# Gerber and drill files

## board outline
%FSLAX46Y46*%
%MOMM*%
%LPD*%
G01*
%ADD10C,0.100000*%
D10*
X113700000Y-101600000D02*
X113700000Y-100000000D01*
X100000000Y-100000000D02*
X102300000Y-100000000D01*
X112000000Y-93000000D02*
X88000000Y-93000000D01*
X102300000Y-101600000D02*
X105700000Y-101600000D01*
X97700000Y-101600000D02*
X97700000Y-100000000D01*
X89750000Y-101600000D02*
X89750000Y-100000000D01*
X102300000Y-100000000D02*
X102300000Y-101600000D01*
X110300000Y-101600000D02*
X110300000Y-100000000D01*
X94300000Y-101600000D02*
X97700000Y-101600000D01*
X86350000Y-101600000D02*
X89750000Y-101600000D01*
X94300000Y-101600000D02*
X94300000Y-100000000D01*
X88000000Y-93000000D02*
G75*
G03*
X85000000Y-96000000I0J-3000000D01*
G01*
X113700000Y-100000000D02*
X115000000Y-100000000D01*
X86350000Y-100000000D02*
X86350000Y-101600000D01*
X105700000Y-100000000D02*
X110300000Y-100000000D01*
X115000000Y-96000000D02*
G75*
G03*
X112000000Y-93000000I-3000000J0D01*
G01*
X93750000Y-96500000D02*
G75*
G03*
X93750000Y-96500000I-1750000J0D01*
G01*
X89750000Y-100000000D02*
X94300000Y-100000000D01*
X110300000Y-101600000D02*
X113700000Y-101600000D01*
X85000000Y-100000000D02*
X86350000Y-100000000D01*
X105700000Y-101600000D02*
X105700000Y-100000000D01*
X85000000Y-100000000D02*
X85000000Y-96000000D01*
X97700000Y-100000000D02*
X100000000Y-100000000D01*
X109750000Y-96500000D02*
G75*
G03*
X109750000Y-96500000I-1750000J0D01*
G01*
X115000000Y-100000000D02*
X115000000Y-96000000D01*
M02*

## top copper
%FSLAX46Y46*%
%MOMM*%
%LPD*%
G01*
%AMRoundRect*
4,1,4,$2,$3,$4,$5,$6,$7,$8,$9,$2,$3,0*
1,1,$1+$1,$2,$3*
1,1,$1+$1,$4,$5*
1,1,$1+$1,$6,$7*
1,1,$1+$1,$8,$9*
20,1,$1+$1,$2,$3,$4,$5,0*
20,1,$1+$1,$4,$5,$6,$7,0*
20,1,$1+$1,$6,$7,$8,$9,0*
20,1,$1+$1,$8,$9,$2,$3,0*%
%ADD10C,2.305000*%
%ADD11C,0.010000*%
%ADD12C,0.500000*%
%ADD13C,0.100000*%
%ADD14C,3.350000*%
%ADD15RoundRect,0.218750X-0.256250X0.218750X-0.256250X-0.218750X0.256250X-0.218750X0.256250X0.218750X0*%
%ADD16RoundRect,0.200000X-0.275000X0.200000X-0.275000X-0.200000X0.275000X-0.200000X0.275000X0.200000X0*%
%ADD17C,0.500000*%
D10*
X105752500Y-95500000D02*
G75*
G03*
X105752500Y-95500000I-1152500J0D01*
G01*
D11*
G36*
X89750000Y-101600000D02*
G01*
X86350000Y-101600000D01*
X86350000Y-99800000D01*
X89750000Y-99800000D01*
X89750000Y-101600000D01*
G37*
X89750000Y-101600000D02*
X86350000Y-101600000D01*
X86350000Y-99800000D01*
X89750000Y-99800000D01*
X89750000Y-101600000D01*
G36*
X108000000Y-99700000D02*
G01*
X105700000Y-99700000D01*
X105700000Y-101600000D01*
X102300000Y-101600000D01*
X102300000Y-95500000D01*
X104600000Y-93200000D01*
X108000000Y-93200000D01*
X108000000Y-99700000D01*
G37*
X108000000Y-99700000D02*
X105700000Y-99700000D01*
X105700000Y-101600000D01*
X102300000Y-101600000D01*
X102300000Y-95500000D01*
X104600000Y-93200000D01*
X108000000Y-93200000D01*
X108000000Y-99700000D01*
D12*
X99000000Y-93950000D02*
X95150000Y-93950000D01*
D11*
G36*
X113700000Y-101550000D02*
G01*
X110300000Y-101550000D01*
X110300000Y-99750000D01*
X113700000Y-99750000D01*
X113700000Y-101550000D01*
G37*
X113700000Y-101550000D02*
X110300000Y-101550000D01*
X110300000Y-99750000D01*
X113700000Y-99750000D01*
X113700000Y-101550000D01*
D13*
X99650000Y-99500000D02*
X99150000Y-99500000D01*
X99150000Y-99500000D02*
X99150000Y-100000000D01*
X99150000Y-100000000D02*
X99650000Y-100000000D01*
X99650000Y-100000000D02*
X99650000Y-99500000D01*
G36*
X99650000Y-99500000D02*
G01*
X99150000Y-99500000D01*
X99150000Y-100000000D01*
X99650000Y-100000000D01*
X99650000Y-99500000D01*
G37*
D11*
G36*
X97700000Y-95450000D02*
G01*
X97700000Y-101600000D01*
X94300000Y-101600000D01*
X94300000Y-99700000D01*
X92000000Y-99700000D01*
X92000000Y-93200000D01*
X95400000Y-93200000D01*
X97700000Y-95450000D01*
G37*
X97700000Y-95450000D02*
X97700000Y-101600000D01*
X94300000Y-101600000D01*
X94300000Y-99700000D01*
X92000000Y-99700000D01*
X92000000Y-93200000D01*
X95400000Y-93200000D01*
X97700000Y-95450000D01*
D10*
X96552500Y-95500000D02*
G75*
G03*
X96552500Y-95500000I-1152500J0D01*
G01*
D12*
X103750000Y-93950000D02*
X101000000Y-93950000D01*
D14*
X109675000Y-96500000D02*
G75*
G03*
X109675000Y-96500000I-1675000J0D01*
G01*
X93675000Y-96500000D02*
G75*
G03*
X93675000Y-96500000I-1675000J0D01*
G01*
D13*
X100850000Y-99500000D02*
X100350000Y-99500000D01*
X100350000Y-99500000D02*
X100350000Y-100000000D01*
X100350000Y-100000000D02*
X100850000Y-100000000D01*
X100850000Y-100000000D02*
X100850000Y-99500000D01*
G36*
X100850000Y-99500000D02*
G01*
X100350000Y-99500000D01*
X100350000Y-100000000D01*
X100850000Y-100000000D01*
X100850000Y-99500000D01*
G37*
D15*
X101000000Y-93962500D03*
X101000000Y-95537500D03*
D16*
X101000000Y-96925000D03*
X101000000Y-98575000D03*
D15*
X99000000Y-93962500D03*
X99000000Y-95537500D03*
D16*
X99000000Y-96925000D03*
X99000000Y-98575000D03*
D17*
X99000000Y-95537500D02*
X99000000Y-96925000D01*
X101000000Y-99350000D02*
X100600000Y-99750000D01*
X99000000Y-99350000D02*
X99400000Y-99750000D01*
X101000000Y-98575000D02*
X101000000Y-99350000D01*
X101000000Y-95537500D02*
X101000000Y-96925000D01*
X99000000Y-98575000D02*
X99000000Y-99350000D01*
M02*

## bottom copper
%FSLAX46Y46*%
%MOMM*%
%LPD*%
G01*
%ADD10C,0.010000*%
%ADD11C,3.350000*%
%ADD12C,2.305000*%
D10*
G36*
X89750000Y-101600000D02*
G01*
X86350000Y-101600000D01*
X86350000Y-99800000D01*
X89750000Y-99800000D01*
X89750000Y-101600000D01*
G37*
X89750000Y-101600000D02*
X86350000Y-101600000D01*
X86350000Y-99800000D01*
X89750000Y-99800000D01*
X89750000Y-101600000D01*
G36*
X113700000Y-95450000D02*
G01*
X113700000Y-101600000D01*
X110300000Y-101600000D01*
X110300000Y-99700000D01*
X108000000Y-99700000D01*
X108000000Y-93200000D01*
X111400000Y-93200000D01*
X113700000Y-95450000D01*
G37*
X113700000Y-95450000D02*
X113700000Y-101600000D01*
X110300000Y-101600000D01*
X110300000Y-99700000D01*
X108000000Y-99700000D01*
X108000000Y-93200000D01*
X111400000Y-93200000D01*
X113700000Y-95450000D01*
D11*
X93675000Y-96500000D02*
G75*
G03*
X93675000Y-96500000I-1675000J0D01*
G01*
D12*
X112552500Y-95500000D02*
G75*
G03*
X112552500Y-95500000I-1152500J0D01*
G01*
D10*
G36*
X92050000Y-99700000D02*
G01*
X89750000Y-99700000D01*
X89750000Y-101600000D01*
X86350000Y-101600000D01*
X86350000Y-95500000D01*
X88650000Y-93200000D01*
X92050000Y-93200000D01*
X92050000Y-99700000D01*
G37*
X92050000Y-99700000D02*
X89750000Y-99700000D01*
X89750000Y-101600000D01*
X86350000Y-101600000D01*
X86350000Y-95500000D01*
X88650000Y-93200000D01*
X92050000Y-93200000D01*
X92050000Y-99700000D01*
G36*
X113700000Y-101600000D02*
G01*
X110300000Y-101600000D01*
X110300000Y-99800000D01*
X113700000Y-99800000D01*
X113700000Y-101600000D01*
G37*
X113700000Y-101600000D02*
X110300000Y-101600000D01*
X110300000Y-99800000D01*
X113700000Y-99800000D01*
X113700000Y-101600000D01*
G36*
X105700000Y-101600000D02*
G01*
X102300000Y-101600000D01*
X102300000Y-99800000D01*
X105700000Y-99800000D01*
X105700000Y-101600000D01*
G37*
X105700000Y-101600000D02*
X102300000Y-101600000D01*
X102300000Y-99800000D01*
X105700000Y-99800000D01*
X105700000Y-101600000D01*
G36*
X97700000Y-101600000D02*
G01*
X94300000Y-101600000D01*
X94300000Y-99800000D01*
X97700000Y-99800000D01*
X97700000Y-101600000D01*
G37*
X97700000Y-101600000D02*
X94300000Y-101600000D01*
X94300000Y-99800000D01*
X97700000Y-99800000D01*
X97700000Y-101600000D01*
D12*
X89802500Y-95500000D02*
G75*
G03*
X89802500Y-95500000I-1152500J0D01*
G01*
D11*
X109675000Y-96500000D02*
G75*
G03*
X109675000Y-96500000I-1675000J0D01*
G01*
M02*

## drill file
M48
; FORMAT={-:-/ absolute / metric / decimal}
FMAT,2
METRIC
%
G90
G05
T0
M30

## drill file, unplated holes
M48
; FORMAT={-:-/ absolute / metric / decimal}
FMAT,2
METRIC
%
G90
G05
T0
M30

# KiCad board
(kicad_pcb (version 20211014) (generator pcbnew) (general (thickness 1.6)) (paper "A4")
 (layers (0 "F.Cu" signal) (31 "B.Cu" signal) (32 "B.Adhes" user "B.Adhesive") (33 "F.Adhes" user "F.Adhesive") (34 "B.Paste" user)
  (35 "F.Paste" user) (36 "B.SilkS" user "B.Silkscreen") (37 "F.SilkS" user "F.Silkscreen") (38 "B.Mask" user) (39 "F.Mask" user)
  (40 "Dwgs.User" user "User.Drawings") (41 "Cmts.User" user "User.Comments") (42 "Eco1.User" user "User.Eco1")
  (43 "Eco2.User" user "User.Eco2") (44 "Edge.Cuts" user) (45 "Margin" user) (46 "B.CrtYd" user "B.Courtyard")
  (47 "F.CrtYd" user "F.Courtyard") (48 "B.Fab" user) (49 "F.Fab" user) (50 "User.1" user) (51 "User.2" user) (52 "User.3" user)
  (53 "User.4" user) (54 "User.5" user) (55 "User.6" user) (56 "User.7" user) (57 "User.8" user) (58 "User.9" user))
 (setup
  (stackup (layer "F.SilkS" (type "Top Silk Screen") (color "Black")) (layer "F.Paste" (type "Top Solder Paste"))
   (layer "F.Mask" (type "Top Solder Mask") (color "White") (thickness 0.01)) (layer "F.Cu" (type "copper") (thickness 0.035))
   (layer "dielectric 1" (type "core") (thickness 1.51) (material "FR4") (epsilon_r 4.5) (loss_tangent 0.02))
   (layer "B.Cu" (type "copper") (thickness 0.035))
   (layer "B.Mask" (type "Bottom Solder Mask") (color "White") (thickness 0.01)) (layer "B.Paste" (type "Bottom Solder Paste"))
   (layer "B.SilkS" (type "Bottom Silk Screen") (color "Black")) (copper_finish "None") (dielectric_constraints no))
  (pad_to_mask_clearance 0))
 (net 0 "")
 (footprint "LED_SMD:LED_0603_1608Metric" (layer "F.Cu") (at 101 94.75 -90)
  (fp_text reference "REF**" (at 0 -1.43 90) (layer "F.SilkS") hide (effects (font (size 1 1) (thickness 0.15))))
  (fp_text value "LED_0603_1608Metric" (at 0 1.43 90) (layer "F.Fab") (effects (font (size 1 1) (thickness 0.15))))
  (pad "1" smd roundrect (at -0.7875 0 270) (size 0.875 0.95) (layers "F.Cu" "F.Paste" "F.Mask") (roundrect_rratio 0.25))
  (pad "2" smd roundrect (at 0.7875 0 270) (size 0.875 0.95) (layers "F.Cu" "F.Paste" "F.Mask") (roundrect_rratio 0.25)))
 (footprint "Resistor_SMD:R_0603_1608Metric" (layer "F.Cu") (at 101 97.75 -90)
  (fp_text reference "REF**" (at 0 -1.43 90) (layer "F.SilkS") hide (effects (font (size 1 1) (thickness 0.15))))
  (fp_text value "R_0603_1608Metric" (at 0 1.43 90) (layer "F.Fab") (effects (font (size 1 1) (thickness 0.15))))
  (pad "1" smd roundrect (at -0.825 0 270) (size 0.8 0.95) (layers "F.Cu" "F.Paste" "F.Mask") (roundrect_rratio 0.25))
  (pad "2" smd roundrect (at 0.825 0 270) (size 0.8 0.95) (layers "F.Cu" "F.Paste" "F.Mask") (roundrect_rratio 0.25)))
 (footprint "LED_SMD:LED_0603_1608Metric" (layer "F.Cu") (at 99 94.75 -90)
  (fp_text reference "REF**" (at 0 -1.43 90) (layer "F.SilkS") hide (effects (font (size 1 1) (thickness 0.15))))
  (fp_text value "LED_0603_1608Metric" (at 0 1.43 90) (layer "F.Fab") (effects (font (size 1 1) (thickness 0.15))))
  (pad "1" smd roundrect (at -0.7875 0 270) (size 0.875 0.95) (layers "F.Cu" "F.Paste" "F.Mask") (roundrect_rratio 0.25))
  (pad "2" smd roundrect (at 0.7875 0 270) (size 0.875 0.95) (layers "F.Cu" "F.Paste" "F.Mask") (roundrect_rratio 0.25)))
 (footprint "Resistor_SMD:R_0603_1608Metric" (layer "F.Cu") (at 99 97.75 -90)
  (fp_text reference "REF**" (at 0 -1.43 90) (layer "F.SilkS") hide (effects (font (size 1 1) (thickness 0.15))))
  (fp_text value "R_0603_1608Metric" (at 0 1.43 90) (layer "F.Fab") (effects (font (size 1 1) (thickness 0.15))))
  (pad "1" smd roundrect (at -0.825 0 270) (size 0.8 0.95) (layers "F.Cu" "F.Paste" "F.Mask") (roundrect_rratio 0.25))
  (pad "2" smd roundrect (at 0.825 0 270) (size 0.8 0.95) (layers "F.Cu" "F.Paste" "F.Mask") (roundrect_rratio 0.25)))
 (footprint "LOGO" (layer "B.Cu") (at 113.250498 96.383565 -160)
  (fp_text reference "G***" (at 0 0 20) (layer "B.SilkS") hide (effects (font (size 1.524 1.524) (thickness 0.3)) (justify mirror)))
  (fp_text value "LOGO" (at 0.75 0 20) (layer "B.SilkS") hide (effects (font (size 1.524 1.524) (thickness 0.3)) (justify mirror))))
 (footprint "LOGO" (layer "B.Cu") (at 97.4 95.15 150)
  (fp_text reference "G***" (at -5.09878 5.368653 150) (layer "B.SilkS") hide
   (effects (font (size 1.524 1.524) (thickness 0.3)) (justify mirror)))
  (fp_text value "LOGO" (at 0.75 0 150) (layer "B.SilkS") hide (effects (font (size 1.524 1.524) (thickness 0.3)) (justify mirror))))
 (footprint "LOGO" (layer "B.Cu") (at 112.5 98.259215 -160)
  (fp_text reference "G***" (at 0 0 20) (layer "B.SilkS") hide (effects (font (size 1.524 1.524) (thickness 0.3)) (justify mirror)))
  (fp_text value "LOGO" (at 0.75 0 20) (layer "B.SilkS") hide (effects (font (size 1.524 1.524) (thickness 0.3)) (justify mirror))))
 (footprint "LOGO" (layer "B.Cu") (at 102.55 96.6 180)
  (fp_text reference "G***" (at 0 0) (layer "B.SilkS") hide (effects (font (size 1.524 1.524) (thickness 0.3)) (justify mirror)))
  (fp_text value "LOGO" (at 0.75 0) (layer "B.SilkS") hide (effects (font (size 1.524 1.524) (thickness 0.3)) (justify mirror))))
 (gr_circle (center 104.6 95.5) (end 106.9 95.5) (layer "F.Cu") (width 0.01) (fill solid))
 (gr_poly (pts (xy 89.75 99.8) (xy 86.35 99.8) (xy 86.35 101.6) (xy 89.75 101.6)) (layer "F.Cu") (width 0.01) (fill solid))
 (gr_poly
  (pts (xy 108 99.7) (xy 105.7 99.7) (xy 105.7 101.6) (xy 102.3 101.6) (xy 102.3 95.5) (xy 104.6 93.2) (xy 108 93.2)) (layer "F.Cu")
  (width 0.01) (fill solid))
 (gr_line (start 99 93.95) (end 95.15 93.95) (layer "F.Cu") (width 0.5))
 (gr_poly (pts (xy 113.7 99.75) (xy 110.3 99.75) (xy 110.3 101.55) (xy 113.7 101.55)) (layer "F.Cu") (width 0.01) (fill solid))
 (gr_rect (start 99.65 99.5) (end 99.15 100) (layer "F.Cu") (width 0.1) (fill solid))
 (gr_poly
  (pts (xy 95.4 93.2) (xy 97.7 95.45) (xy 97.7 101.6) (xy 94.3 101.6) (xy 94.3 99.7) (xy 92 99.7) (xy 92 93.2)) (layer "F.Cu") (width 0.01)
  (fill solid))
 (gr_circle (center 95.4 95.5) (end 97.7 95.5) (layer "F.Cu") (width 0.01) (fill solid))
 (gr_line (start 103.75 93.95) (end 101 93.95) (layer "F.Cu") (width 0.5))
 (gr_circle (center 108 96.5) (end 111.3 96.5) (layer "F.Cu") (width 0.1) (fill solid))
 (gr_circle (center 92 96.5) (end 88.7 96.5) (layer "F.Cu") (width 0.1) (fill solid))
 (gr_rect (start 100.85 99.5) (end 100.35 100) (layer "F.Cu") (width 0.1) (fill solid))
 (gr_poly (pts (xy 86.35 99.8) (xy 89.75 99.8) (xy 89.75 101.6) (xy 86.35 101.6)) (layer "B.Cu") (width 0.01) (fill solid))
 (gr_poly
  (pts (xy 111.4 93.2) (xy 113.7 95.45) (xy 113.7 101.6) (xy 110.3 101.6) (xy 110.3 99.7) (xy 108 99.7) (xy 108 93.2)) (layer "B.Cu")
  (width 0.01) (fill solid))
 (gr_circle (center 92 96.5) (end 88.7 96.5) (layer "B.Cu") (width 0.1) (fill solid))
 (gr_circle (center 111.4 95.5) (end 109.1 95.5) (layer "B.Cu") (width 0.01) (fill solid))
 (gr_poly
  (pts (xy 92.05 99.7) (xy 89.75 99.7) (xy 89.75 101.6) (xy 86.35 101.6) (xy 86.35 95.5) (xy 88.65 93.2) (xy 92.05 93.2)) (layer "B.Cu")
  (width 0.01) (fill solid))
 (gr_poly (pts (xy 110.3 99.8) (xy 113.7 99.8) (xy 113.7 101.6) (xy 110.3 101.6)) (layer "B.Cu") (width 0.01) (fill solid))
 (gr_poly (pts (xy 102.3 99.8) (xy 105.7 99.8) (xy 105.7 101.6) (xy 102.3 101.6)) (layer "B.Cu") (width 0.01) (fill solid))
 (gr_poly (pts (xy 94.3 99.8) (xy 97.7 99.8) (xy 97.7 101.6) (xy 94.3 101.6)) (layer "B.Cu") (width 0.01) (fill solid))
 (gr_circle (center 88.65 95.5) (end 86.35 95.5) (layer "B.Cu") (width 0.01) (fill solid))
 (gr_circle (center 108 96.5) (end 111.3 96.5) (layer "B.Cu") (width 0.1) (fill solid))
 (gr_line (start 113.7 101.6) (end 113.7 100) (layer "Edge.Cuts") (width 0.1))
 (gr_line (start 100 100) (end 102.3 100) (layer "Edge.Cuts") (width 0.1))
 (gr_line (start 112 93) (end 88 93) (layer "Edge.Cuts") (width 0.1))
 (gr_line (start 102.3 101.6) (end 105.7 101.6) (layer "Edge.Cuts") (width 0.1))
 (gr_line (start 97.7 101.6) (end 97.7 100) (layer "Edge.Cuts") (width 0.1))
 (gr_line (start 89.75 101.6) (end 89.75 100) (layer "Edge.Cuts") (width 0.1))
 (gr_line (start 102.3 100) (end 102.3 101.6) (layer "Edge.Cuts") (width 0.1))
 (gr_line (start 110.3 101.6) (end 110.3 100) (layer "Edge.Cuts") (width 0.1))
 (gr_line (start 94.3 101.6) (end 97.7 101.6) (layer "Edge.Cuts") (width 0.1))
 (gr_line (start 86.35 101.6) (end 89.75 101.6) (layer "Edge.Cuts") (width 0.1))
 (gr_line (start 94.3 101.6) (end 94.3 100) (layer "Edge.Cuts") (width 0.1))
 (gr_arc (start 85 96) (mid 85.87868 93.87868) (end 88 93) (layer "Edge.Cuts") (width 0.1))
 (gr_line (start 113.7 100) (end 115 100) (layer "Edge.Cuts") (width 0.1))
 (gr_line (start 86.35 100) (end 86.35 101.6) (layer "Edge.Cuts") (width 0.1))
 (gr_line (start 105.7 100) (end 110.3 100) (layer "Edge.Cuts") (width 0.1))
 (gr_arc (start 112 93) (mid 114.12132 93.87868) (end 115 96) (layer "Edge.Cuts") (width 0.1))
 (gr_circle (center 92 96.5) (end 93.75 96.5) (layer "Edge.Cuts") (width 0.1) (fill none))
 (gr_line (start 89.75 100) (end 94.3 100) (layer "Edge.Cuts") (width 0.1))
 (gr_line (start 110.3 101.6) (end 113.7 101.6) (layer "Edge.Cuts") (width 0.1))
 (gr_line (start 85 100) (end 86.35 100) (layer "Edge.Cuts") (width 0.1))
 (gr_line (start 105.7 101.6) (end 105.7 100) (layer "Edge.Cuts") (width 0.1))
 (gr_line (start 85 100) (end 85 96) (layer "Edge.Cuts") (width 0.1))
 (gr_line (start 97.7 100) (end 100 100) (layer "Edge.Cuts") (width 0.1))
 (gr_circle (center 108 96.5) (end 109.75 96.5) (layer "Edge.Cuts") (width 0.1) (fill none))
 (gr_line (start 115 100) (end 115 96) (layer "Edge.Cuts") (width 0.1))
 (segment (start 99 95.5375) (end 99 96.925) (width 0.5) (layer "F.Cu") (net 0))
 (segment (start 101 99.35) (end 100.6 99.75) (width 0.5) (layer "F.Cu") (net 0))
 (segment (start 99 99.35) (end 99.4 99.75) (width 0.5) (layer "F.Cu") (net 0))
 (segment (start 101 98.575) (end 101 99.35) (width 0.5) (layer "F.Cu") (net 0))
 (segment (start 101 95.5375) (end 101 96.925) (width 0.5) (layer "F.Cu") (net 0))
 (segment (start 99 98.575) (end 99 99.35) (width 0.5) (layer "F.Cu") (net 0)))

